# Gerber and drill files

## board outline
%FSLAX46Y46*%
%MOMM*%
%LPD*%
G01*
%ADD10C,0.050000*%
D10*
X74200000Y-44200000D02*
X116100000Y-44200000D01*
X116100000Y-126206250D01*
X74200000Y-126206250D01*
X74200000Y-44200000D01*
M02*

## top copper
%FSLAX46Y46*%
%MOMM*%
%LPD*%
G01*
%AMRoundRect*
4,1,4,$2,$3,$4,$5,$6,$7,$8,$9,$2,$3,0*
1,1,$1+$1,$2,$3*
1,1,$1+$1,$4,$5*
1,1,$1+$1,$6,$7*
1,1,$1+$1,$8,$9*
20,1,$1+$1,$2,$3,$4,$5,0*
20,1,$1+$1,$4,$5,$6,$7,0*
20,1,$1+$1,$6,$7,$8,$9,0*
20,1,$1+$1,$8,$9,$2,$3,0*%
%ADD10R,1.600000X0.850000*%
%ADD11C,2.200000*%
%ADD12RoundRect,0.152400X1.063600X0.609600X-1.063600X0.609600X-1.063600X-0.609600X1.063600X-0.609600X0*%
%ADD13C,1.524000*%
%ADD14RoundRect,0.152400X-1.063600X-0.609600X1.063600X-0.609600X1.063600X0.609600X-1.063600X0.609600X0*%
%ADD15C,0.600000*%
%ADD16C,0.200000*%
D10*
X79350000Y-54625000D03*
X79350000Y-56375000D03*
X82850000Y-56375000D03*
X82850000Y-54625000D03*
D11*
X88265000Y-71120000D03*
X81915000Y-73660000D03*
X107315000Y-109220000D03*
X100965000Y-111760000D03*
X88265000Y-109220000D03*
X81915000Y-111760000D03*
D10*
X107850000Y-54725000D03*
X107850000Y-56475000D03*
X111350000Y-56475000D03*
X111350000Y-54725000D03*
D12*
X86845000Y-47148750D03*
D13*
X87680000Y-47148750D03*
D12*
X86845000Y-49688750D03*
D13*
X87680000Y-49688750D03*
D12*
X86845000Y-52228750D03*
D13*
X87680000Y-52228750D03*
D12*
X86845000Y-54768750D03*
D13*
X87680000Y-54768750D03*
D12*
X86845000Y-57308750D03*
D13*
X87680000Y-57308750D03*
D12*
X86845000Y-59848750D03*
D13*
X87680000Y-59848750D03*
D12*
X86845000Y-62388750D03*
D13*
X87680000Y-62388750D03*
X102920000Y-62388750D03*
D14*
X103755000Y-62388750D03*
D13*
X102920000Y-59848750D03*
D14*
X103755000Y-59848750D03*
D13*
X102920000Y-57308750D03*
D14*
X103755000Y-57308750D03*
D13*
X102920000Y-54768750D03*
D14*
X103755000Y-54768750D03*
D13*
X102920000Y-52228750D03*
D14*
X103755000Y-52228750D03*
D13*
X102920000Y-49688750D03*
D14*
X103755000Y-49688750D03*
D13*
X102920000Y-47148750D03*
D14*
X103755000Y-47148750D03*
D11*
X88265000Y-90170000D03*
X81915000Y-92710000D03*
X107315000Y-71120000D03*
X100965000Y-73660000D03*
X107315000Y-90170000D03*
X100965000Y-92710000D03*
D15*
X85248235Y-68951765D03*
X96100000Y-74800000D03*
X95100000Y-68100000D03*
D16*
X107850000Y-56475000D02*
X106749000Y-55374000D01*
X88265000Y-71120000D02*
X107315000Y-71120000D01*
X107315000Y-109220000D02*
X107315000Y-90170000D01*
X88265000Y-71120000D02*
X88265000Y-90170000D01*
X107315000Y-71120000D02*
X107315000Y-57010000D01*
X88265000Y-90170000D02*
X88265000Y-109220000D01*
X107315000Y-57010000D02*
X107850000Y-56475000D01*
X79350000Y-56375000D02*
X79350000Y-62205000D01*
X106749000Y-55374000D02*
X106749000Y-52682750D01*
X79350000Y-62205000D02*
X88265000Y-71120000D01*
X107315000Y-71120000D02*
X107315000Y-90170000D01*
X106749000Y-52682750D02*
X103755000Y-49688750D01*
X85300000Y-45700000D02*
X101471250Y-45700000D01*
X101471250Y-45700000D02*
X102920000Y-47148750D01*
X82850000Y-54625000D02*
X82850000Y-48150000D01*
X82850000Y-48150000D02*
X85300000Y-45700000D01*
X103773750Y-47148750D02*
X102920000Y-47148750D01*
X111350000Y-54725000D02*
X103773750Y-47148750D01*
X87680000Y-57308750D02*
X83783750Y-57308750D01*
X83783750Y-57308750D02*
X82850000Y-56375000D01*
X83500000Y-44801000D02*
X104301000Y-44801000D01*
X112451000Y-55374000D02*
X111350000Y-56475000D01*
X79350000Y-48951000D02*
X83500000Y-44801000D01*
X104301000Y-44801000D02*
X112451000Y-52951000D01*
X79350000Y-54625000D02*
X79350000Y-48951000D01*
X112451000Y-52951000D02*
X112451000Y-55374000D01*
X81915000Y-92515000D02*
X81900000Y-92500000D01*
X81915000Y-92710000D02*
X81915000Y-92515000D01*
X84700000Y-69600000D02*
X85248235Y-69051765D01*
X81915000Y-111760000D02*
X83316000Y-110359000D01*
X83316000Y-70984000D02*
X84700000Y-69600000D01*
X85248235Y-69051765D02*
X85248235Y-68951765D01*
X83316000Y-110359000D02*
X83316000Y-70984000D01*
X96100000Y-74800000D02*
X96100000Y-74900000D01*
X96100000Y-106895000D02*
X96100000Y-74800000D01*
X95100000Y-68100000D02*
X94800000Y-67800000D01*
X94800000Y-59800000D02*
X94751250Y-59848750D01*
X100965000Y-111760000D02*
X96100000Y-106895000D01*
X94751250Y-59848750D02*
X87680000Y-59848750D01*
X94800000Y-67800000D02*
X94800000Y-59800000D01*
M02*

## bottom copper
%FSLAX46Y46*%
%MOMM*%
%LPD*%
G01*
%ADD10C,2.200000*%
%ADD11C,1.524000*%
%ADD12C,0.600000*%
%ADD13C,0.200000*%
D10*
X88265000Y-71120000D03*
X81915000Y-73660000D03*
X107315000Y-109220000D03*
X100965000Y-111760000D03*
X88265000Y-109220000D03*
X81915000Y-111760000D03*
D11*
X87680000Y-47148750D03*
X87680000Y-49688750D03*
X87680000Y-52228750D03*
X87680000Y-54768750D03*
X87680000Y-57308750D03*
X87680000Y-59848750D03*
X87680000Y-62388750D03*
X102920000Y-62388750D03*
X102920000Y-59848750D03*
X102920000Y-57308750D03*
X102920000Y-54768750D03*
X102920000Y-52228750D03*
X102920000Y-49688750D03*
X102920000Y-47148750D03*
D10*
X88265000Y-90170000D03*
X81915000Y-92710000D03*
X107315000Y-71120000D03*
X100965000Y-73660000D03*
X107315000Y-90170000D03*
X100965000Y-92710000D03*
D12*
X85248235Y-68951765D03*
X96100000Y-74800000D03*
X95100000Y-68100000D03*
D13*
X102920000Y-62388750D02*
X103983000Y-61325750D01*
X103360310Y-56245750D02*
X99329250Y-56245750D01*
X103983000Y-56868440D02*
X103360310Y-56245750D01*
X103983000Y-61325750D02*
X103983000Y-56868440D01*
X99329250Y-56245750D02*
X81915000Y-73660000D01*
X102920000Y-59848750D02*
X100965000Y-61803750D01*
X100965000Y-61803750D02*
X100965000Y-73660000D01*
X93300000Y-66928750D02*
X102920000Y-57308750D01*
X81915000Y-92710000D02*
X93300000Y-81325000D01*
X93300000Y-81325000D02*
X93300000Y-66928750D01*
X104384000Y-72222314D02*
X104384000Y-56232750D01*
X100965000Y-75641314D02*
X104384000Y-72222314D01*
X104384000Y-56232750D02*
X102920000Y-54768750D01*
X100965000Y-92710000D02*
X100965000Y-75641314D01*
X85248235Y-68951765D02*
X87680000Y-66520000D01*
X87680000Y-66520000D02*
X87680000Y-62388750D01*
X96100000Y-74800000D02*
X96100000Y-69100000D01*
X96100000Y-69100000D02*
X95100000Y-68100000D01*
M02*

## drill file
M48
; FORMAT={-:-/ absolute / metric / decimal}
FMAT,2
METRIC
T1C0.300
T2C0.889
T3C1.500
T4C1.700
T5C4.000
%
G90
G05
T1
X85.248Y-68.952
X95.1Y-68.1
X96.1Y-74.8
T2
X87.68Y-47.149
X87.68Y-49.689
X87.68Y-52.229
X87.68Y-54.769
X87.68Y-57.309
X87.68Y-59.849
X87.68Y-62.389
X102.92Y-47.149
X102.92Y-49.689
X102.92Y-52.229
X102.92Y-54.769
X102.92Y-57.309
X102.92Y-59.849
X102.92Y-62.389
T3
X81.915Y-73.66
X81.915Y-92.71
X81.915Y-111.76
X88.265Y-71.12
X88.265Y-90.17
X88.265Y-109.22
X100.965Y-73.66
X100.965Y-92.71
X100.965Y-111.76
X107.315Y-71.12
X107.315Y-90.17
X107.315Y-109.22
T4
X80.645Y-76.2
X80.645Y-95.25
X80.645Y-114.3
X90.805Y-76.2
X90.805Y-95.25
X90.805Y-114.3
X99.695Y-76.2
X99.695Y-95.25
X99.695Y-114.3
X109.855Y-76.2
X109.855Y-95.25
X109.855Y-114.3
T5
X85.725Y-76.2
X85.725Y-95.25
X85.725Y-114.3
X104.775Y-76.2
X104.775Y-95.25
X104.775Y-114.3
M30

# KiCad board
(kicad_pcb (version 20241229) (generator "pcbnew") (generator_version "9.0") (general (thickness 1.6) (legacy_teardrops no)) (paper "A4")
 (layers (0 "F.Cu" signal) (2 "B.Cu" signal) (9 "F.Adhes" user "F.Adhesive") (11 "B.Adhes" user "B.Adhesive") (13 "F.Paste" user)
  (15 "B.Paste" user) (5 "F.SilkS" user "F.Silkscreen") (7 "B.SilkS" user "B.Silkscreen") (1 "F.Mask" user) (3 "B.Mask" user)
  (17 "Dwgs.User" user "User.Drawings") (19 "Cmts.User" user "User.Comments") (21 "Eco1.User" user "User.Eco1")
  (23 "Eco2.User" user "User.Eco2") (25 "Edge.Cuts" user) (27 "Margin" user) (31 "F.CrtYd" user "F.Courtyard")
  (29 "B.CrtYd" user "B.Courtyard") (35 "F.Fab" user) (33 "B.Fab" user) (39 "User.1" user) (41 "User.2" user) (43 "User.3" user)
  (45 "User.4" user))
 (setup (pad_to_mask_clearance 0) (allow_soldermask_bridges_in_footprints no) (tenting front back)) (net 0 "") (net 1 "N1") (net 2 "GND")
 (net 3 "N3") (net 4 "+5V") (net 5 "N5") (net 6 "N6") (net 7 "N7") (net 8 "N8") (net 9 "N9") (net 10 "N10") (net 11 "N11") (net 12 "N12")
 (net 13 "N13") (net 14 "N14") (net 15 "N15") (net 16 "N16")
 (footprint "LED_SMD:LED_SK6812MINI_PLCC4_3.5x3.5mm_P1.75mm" (layer "F.Cu") (at 81.1 55.5)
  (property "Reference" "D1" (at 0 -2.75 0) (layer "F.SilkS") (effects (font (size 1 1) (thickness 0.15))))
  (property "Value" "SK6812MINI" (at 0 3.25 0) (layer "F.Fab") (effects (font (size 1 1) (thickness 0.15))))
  (pad "1" smd rect (at -1.75 -0.875) (size 1.6 0.85) (layers "F.Cu" "F.Mask" "F.Paste") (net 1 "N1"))
  (pad "2" smd rect (at -1.75 0.875) (size 1.6 0.85) (layers "F.Cu" "F.Mask" "F.Paste") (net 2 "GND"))
  (pad "3" smd rect (at 1.75 0.875) (size 1.6 0.85) (layers "F.Cu" "F.Mask" "F.Paste") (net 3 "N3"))
  (pad "4" smd rect (at 1.75 -0.875) (size 1.6 0.85) (layers "F.Cu" "F.Mask" "F.Paste") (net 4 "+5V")))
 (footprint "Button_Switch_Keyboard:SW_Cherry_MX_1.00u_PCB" (layer "F.Cu") (at 88.265 71.12)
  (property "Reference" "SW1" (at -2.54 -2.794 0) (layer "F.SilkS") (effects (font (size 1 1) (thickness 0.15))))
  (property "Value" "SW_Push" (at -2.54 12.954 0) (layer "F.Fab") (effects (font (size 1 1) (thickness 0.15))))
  (pad "" np_thru_hole circle (at -7.62 5.08) (size 1.7 1.7) (drill 1.7) (layers "*.Cu" "*.Mask"))
  (pad "" np_thru_hole circle (at -2.54 5.08) (size 4 4) (drill 4) (layers "*.Cu" "*.Mask"))
  (pad "" np_thru_hole circle (at 2.54 5.08) (size 1.7 1.7) (drill 1.7) (layers "*.Cu" "*.Mask"))
  (pad "1" thru_hole circle (at 0 0) (size 2.2 2.2) (drill 1.5) (layers "*.Cu" "*.Mask") (remove_unused_layers no) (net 2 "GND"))
  (pad "2" thru_hole circle (at -6.35 2.54) (size 2.2 2.2) (drill 1.5) (layers "*.Cu" "*.Mask") (remove_unused_layers no) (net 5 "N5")))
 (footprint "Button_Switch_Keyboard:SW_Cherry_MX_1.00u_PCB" (layer "F.Cu") (at 107.315 109.22)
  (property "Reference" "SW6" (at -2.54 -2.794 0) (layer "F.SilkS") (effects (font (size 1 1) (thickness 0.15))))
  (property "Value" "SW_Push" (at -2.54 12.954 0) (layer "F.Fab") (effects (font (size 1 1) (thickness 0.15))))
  (pad "" np_thru_hole circle (at -7.62 5.08) (size 1.7 1.7) (drill 1.7) (layers "*.Cu" "*.Mask"))
  (pad "" np_thru_hole circle (at -2.54 5.08) (size 4 4) (drill 4) (layers "*.Cu" "*.Mask"))
  (pad "" np_thru_hole circle (at 2.54 5.08) (size 1.7 1.7) (drill 1.7) (layers "*.Cu" "*.Mask"))
  (pad "1" thru_hole circle (at 0 0) (size 2.2 2.2) (drill 1.5) (layers "*.Cu" "*.Mask") (remove_unused_layers no) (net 2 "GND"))
  (pad "2" thru_hole circle (at -6.35 2.54) (size 2.2 2.2) (drill 1.5) (layers "*.Cu" "*.Mask") (remove_unused_layers no) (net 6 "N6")))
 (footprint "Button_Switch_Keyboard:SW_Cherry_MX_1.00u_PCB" (layer "F.Cu") (at 88.265 109.22)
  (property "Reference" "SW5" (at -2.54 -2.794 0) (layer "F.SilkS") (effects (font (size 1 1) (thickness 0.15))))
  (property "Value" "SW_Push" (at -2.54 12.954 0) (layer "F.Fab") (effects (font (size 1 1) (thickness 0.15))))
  (pad "" np_thru_hole circle (at -7.62 5.08) (size 1.7 1.7) (drill 1.7) (layers "*.Cu" "*.Mask"))
  (pad "" np_thru_hole circle (at -2.54 5.08) (size 4 4) (drill 4) (layers "*.Cu" "*.Mask"))
  (pad "" np_thru_hole circle (at 2.54 5.08) (size 1.7 1.7) (drill 1.7) (layers "*.Cu" "*.Mask"))
  (pad "1" thru_hole circle (at 0 0) (size 2.2 2.2) (drill 1.5) (layers "*.Cu" "*.Mask") (remove_unused_layers no) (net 2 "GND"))
  (pad "2" thru_hole circle (at -6.35 2.54) (size 2.2 2.2) (drill 1.5) (layers "*.Cu" "*.Mask") (remove_unused_layers no) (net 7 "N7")))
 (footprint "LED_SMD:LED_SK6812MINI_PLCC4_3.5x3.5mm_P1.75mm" (layer "F.Cu") (at 109.6 55.6)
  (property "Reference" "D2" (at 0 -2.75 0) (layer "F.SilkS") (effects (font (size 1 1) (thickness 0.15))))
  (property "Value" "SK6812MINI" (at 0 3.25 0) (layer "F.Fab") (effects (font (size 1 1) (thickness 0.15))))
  (pad "1" smd rect (at -1.75 -0.875) (size 1.6 0.85) (layers "F.Cu" "F.Mask" "F.Paste") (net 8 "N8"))
  (pad "2" smd rect (at -1.75 0.875) (size 1.6 0.85) (layers "F.Cu" "F.Mask" "F.Paste") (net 2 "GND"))
  (pad "3" smd rect (at 1.75 0.875) (size 1.6 0.85) (layers "F.Cu" "F.Mask" "F.Paste") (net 1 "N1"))
  (pad "4" smd rect (at 1.75 -0.875) (size 1.6 0.85) (layers "F.Cu" "F.Mask" "F.Paste") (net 4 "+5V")))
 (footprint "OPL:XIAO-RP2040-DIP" (layer "F.Cu") (at 95.3 54.76875)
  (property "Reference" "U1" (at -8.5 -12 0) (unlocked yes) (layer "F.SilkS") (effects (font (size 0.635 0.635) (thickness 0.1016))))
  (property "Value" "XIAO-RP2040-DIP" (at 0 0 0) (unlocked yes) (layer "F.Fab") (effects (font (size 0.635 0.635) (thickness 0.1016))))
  (pad "1" smd roundrect (at -8.455 -7.62 180) (size 2.432 1.524) (layers "F.Cu" "F.Mask") (roundrect_rratio 0.1) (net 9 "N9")
   (thermal_bridge_angle 45))
  (pad "1" thru_hole circle (at -7.62 -7.62 180) (size 1.524 1.524) (drill 0.889) (layers "*.Cu" "*.Mask") (remove_unused_layers no)
   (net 9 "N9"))
  (pad "2" smd roundrect (at -8.455 -5.08 180) (size 2.432 1.524) (layers "F.Cu" "F.Mask") (roundrect_rratio 0.1) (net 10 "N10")
   (thermal_bridge_angle 45))
  (pad "2" thru_hole circle (at -7.62 -5.08 180) (size 1.524 1.524) (drill 0.889) (layers "*.Cu" "*.Mask") (remove_unused_layers no)
   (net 10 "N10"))
  (pad "3" smd roundrect (at -8.455 -2.54 180) (size 2.432 1.524) (layers "F.Cu" "F.Mask") (roundrect_rratio 0.1) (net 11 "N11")
   (thermal_bridge_angle 45))
  (pad "3" thru_hole circle (at -7.62 -2.54 180) (size 1.524 1.524) (drill 0.889) (layers "*.Cu" "*.Mask") (remove_unused_layers no)
   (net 11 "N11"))
  (pad "4" smd roundrect (at -8.455 0 180) (size 2.432 1.524) (layers "F.Cu" "F.Mask") (roundrect_rratio 0.1) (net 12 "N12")
   (thermal_bridge_angle 45))
  (pad "4" thru_hole circle (at -7.62 0 180) (size 1.524 1.524) (drill 0.889) (layers "*.Cu" "*.Mask") (remove_unused_layers no)
   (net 12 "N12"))
  (pad "5" smd roundrect (at -8.455 2.54 180) (size 2.432 1.524) (layers "F.Cu" "F.Mask") (roundrect_rratio 0.1) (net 3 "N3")
   (thermal_bridge_angle 45))
  (pad "5" thru_hole circle (at -7.62 2.54 180) (size 1.524 1.524) (drill 0.889) (layers "*.Cu" "*.Mask") (remove_unused_layers no)
   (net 3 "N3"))
  (pad "6" smd roundrect (at -8.455 5.08 180) (size 2.432 1.524) (layers "F.Cu" "F.Mask") (roundrect_rratio 0.1) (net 6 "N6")
   (thermal_bridge_angle 45))
  (pad "6" thru_hole circle (at -7.62 5.08 180) (size 1.524 1.524) (drill 0.889) (layers "*.Cu" "*.Mask") (remove_unused_layers no)
   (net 6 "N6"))
  (pad "7" smd roundrect (at -8.455 7.62 180) (size 2.432 1.524) (layers "F.Cu" "F.Mask") (roundrect_rratio 0.1) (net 7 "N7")
   (thermal_bridge_angle 45))
  (pad "7" thru_hole circle (at -7.62 7.62 180) (size 1.524 1.524) (drill 0.889) (layers "*.Cu" "*.Mask") (remove_unused_layers no)
   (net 7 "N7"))
  (pad "8" thru_hole circle (at 7.62 7.62) (size 1.524 1.524) (drill 0.889) (layers "*.Cu" "*.Mask") (remove_unused_layers no) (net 5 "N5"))
  (pad "8" smd roundrect (at 8.455 7.62) (size 2.432 1.524) (layers "F.Cu" "F.Mask") (roundrect_rratio 0.1) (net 5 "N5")
   (thermal_bridge_angle 45))
  (pad "9" thru_hole circle (at 7.62 5.08) (size 1.524 1.524) (drill 0.889) (layers "*.Cu" "*.Mask") (remove_unused_layers no)
   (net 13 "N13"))
  (pad "9" smd roundrect (at 8.455 5.08) (size 2.432 1.524) (layers "F.Cu" "F.Mask") (roundrect_rratio 0.1) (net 13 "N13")
   (thermal_bridge_angle 45))
  (pad "10" thru_hole circle (at 7.62 2.54) (size 1.524 1.524) (drill 0.889) (layers "*.Cu" "*.Mask") (remove_unused_layers no)
   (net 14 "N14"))
  (pad "10" smd roundrect (at 8.455 2.54) (size 2.432 1.524) (layers "F.Cu" "F.Mask") (roundrect_rratio 0.1) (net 14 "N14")
   (thermal_bridge_angle 45))
  (pad "11" thru_hole circle (at 7.62 0) (size 1.524 1.524) (drill 0.889) (layers "*.Cu" "*.Mask") (remove_unused_layers no) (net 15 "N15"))
  (pad "11" smd roundrect (at 8.455 0) (size 2.432 1.524) (layers "F.Cu" "F.Mask") (roundrect_rratio 0.1) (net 15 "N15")
   (thermal_bridge_angle 45))
  (pad "12" thru_hole circle (at 7.62 -2.54) (size 1.524 1.524) (drill 0.889) (layers "*.Cu" "*.Mask") (remove_unused_layers no)
   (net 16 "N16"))
  (pad "12" smd roundrect (at 8.455 -2.54) (size 2.432 1.524) (layers "F.Cu" "F.Mask") (roundrect_rratio 0.1) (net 16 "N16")
   (thermal_bridge_angle 45))
  (pad "13" thru_hole circle (at 7.62 -5.08) (size 1.524 1.524) (drill 0.889) (layers "*.Cu" "*.Mask") (remove_unused_layers no)
   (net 2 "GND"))
  (pad "13" smd roundrect (at 8.455 -5.08) (size 2.432 1.524) (layers "F.Cu" "F.Mask") (roundrect_rratio 0.1) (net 2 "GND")
   (thermal_bridge_angle 45))
  (pad "14" thru_hole circle (at 7.62 -7.62) (size 1.524 1.524) (drill 0.889) (layers "*.Cu" "*.Mask") (remove_unused_layers no)
   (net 4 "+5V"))
  (pad "14" smd roundrect (at 8.455 -7.62) (size 2.432 1.524) (layers "F.Cu" "F.Mask") (roundrect_rratio 0.1) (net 4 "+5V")
   (thermal_bridge_angle 45)))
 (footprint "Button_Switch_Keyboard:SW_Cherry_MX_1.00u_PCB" (layer "F.Cu") (at 88.265 90.17)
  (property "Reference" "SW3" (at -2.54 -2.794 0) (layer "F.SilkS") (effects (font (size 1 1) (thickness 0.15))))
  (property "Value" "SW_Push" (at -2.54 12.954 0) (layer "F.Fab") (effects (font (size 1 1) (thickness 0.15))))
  (pad "" np_thru_hole circle (at -7.62 5.08) (size 1.7 1.7) (drill 1.7) (layers "*.Cu" "*.Mask"))
  (pad "" np_thru_hole circle (at -2.54 5.08) (size 4 4) (drill 4) (layers "*.Cu" "*.Mask"))
  (pad "" np_thru_hole circle (at 2.54 5.08) (size 1.7 1.7) (drill 1.7) (layers "*.Cu" "*.Mask"))
  (pad "1" thru_hole circle (at 0 0) (size 2.2 2.2) (drill 1.5) (layers "*.Cu" "*.Mask") (remove_unused_layers no) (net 2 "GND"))
  (pad "2" thru_hole circle (at -6.35 2.54) (size 2.2 2.2) (drill 1.5) (layers "*.Cu" "*.Mask") (remove_unused_layers no) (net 14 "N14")))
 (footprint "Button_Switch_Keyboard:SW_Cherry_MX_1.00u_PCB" (layer "F.Cu") (at 107.315 71.12)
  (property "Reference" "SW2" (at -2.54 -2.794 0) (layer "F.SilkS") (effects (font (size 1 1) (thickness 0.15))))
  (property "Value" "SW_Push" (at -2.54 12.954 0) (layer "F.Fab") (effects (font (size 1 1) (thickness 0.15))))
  (pad "" np_thru_hole circle (at -7.62 5.08) (size 1.7 1.7) (drill 1.7) (layers "*.Cu" "*.Mask"))
  (pad "" np_thru_hole circle (at -2.54 5.08) (size 4 4) (drill 4) (layers "*.Cu" "*.Mask"))
  (pad "" np_thru_hole circle (at 2.54 5.08) (size 1.7 1.7) (drill 1.7) (layers "*.Cu" "*.Mask"))
  (pad "1" thru_hole circle (at 0 0) (size 2.2 2.2) (drill 1.5) (layers "*.Cu" "*.Mask") (remove_unused_layers no) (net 2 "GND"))
  (pad "2" thru_hole circle (at -6.35 2.54) (size 2.2 2.2) (drill 1.5) (layers "*.Cu" "*.Mask") (remove_unused_layers no) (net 13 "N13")))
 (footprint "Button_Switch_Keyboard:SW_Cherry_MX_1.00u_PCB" (layer "F.Cu") (at 107.315 90.17)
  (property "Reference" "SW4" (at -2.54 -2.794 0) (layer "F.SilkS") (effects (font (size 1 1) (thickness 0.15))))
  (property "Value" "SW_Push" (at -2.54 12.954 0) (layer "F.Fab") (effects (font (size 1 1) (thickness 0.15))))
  (pad "" np_thru_hole circle (at -7.62 5.08) (size 1.7 1.7) (drill 1.7) (layers "*.Cu" "*.Mask"))
  (pad "" np_thru_hole circle (at -2.54 5.08) (size 4 4) (drill 4) (layers "*.Cu" "*.Mask"))
  (pad "" np_thru_hole circle (at 2.54 5.08) (size 1.7 1.7) (drill 1.7) (layers "*.Cu" "*.Mask"))
  (pad "1" thru_hole circle (at 0 0) (size 2.2 2.2) (drill 1.5) (layers "*.Cu" "*.Mask") (remove_unused_layers no) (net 2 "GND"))
  (pad "2" thru_hole circle (at -6.35 2.54) (size 2.2 2.2) (drill 1.5) (layers "*.Cu" "*.Mask") (remove_unused_layers no) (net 15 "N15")))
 (gr_rect (start 74.2 44.2) (end 116.1 126.20625) (stroke (width 0.05) (type default)) (fill no) (layer "Edge.Cuts"))
 (segment (start 107.85 56.475) (end 106.749 55.374) (width 0.2) (layer "F.Cu") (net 2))
 (segment (start 88.265 71.12) (end 107.315 71.12) (width 0.2) (layer "F.Cu") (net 2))
 (segment (start 107.315 109.22) (end 107.315 90.17) (width 0.2) (layer "F.Cu") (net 2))
 (segment (start 88.265 71.12) (end 88.265 90.17) (width 0.2) (layer "F.Cu") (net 2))
 (segment (start 107.315 71.12) (end 107.315 57.01) (width 0.2) (layer "F.Cu") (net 2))
 (segment (start 88.265 90.17) (end 88.265 109.22) (width 0.2) (layer "F.Cu") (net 2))
 (segment (start 107.315 57.01) (end 107.85 56.475) (width 0.2) (layer "F.Cu") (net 2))
 (segment (start 79.35 56.375) (end 79.35 62.205) (width 0.2) (layer "F.Cu") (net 2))
 (segment (start 106.749 55.374) (end 106.749 52.68275) (width 0.2) (layer "F.Cu") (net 2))
 (segment (start 79.35 62.205) (end 88.265 71.12) (width 0.2) (layer "F.Cu") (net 2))
 (segment (start 107.315 71.12) (end 107.315 90.17) (width 0.2) (layer "F.Cu") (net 2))
 (segment (start 106.749 52.68275) (end 103.755 49.68875) (width 0.2) (layer "F.Cu") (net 2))
 (segment (start 85.3 45.7) (end 101.47125 45.7) (width 0.2) (layer "F.Cu") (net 4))
 (segment (start 101.47125 45.7) (end 102.92 47.14875) (width 0.2) (layer "F.Cu") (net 4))
 (segment (start 82.85 54.625) (end 82.85 48.15) (width 0.2) (layer "F.Cu") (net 4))
 (segment (start 82.85 48.15) (end 85.3 45.7) (width 0.2) (layer "F.Cu") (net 4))
 (segment (start 103.77375 47.14875) (end 102.92 47.14875) (width 0.2) (layer "F.Cu") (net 4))
 (segment (start 111.35 54.725) (end 103.77375 47.14875) (width 0.2) (layer "F.Cu") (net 4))
 (segment (start 87.68 57.30875) (end 83.78375 57.30875) (width 0.2) (layer "F.Cu") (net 3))
 (segment (start 83.78375 57.30875) (end 82.85 56.375) (width 0.2) (layer "F.Cu") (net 3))
 (segment (start 83.5 44.801) (end 104.301 44.801) (width 0.2) (layer "F.Cu") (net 1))
 (segment (start 112.451 55.374) (end 111.35 56.475) (width 0.2) (layer "F.Cu") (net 1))
 (segment (start 79.35 48.951) (end 83.5 44.801) (width 0.2) (layer "F.Cu") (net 1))
 (segment (start 104.301 44.801) (end 112.451 52.951) (width 0.2) (layer "F.Cu") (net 1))
 (segment (start 79.35 54.625) (end 79.35 48.951) (width 0.2) (layer "F.Cu") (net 1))
 (segment (start 112.451 52.951) (end 112.451 55.374) (width 0.2) (layer "F.Cu") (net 1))
 (segment (start 102.92 62.38875) (end 103.983 61.32575) (width 0.2) (layer "B.Cu") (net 5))
 (segment (start 103.36031 56.24575) (end 99.32925 56.24575) (width 0.2) (layer "B.Cu") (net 5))
 (segment (start 103.983 56.86844) (end 103.36031 56.24575) (width 0.2) (layer "B.Cu") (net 5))
 (segment (start 103.983 61.32575) (end 103.983 56.86844) (width 0.2) (layer "B.Cu") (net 5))
 (segment (start 99.32925 56.24575) (end 81.915 73.66) (width 0.2) (layer "B.Cu") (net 5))
 (segment (start 102.92 59.84875) (end 100.965 61.80375) (width 0.2) (layer "B.Cu") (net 13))
 (segment (start 100.965 61.80375) (end 100.965 73.66) (width 0.2) (layer "B.Cu") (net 13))
 (segment (start 81.915 92.515) (end 81.9 92.5) (width 0.2) (layer "F.Cu") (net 14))
 (segment (start 81.915 92.71) (end 81.915 92.515) (width 0.2) (layer "F.Cu") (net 14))
 (segment (start 93.3 66.92875) (end 102.92 57.30875) (width 0.2) (layer "B.Cu") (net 14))
 (segment (start 81.915 92.71) (end 93.3 81.325) (width 0.2) (layer "B.Cu") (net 14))
 (segment (start 93.3 81.325) (end 93.3 66.92875) (width 0.2) (layer "B.Cu") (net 14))
 (segment (start 104.384 72.222314) (end 104.384 56.23275) (width 0.2) (layer "B.Cu") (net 15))
 (segment (start 100.965 75.641314) (end 104.384 72.222314) (width 0.2) (layer "B.Cu") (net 15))
 (segment (start 104.384 56.23275) (end 102.92 54.76875) (width 0.2) (layer "B.Cu") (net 15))
 (segment (start 100.965 92.71) (end 100.965 75.641314) (width 0.2) (layer "B.Cu") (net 15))
 (segment (start 84.7 69.6) (end 85.248235 69.051765) (width 0.2) (layer "F.Cu") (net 7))
 (segment (start 81.915 111.76) (end 83.316 110.359) (width 0.2) (layer "F.Cu") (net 7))
 (segment (start 83.316 70.984) (end 84.7 69.6) (width 0.2) (layer "F.Cu") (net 7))
 (segment (start 85.248235 69.051765) (end 85.248235 68.951765) (width 0.2) (layer "F.Cu") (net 7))
 (segment (start 83.316 110.359) (end 83.316 70.984) (width 0.2) (layer "F.Cu") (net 7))
 (via (at 85.248235 68.951765) (size 0.6) (drill 0.3) (layers "F.Cu" "B.Cu") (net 7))
 (segment (start 85.248235 68.951765) (end 87.68 66.52) (width 0.2) (layer "B.Cu") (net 7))
 (segment (start 87.68 66.52) (end 87.68 62.38875) (width 0.2) (layer "B.Cu") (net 7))
 (segment (start 96.1 74.8) (end 96.1 74.9) (width 0.2) (layer "F.Cu") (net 6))
 (segment (start 96.1 106.895) (end 96.1 74.8) (width 0.2) (layer "F.Cu") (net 6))
 (segment (start 95.1 68.1) (end 94.8 67.8) (width 0.2) (layer "F.Cu") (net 6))
 (segment (start 94.8 59.8) (end 94.75125 59.84875) (width 0.2) (layer "F.Cu") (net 6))
 (segment (start 100.965 111.76) (end 96.1 106.895) (width 0.2) (layer "F.Cu") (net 6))
 (segment (start 94.75125 59.84875) (end 87.68 59.84875) (width 0.2) (layer "F.Cu") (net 6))
 (segment (start 94.8 67.8) (end 94.8 59.8) (width 0.2) (layer "F.Cu") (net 6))
 (via (at 96.1 74.8) (size 0.6) (drill 0.3) (layers "F.Cu" "B.Cu") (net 6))
 (via (at 95.1 68.1) (size 0.6) (drill 0.3) (layers "F.Cu" "B.Cu") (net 6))
 (segment (start 96.1 74.8) (end 96.1 69.1) (width 0.2) (layer "B.Cu") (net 6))
 (segment (start 96.1 69.1) (end 95.1 68.1) (width 0.2) (layer "B.Cu") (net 6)))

